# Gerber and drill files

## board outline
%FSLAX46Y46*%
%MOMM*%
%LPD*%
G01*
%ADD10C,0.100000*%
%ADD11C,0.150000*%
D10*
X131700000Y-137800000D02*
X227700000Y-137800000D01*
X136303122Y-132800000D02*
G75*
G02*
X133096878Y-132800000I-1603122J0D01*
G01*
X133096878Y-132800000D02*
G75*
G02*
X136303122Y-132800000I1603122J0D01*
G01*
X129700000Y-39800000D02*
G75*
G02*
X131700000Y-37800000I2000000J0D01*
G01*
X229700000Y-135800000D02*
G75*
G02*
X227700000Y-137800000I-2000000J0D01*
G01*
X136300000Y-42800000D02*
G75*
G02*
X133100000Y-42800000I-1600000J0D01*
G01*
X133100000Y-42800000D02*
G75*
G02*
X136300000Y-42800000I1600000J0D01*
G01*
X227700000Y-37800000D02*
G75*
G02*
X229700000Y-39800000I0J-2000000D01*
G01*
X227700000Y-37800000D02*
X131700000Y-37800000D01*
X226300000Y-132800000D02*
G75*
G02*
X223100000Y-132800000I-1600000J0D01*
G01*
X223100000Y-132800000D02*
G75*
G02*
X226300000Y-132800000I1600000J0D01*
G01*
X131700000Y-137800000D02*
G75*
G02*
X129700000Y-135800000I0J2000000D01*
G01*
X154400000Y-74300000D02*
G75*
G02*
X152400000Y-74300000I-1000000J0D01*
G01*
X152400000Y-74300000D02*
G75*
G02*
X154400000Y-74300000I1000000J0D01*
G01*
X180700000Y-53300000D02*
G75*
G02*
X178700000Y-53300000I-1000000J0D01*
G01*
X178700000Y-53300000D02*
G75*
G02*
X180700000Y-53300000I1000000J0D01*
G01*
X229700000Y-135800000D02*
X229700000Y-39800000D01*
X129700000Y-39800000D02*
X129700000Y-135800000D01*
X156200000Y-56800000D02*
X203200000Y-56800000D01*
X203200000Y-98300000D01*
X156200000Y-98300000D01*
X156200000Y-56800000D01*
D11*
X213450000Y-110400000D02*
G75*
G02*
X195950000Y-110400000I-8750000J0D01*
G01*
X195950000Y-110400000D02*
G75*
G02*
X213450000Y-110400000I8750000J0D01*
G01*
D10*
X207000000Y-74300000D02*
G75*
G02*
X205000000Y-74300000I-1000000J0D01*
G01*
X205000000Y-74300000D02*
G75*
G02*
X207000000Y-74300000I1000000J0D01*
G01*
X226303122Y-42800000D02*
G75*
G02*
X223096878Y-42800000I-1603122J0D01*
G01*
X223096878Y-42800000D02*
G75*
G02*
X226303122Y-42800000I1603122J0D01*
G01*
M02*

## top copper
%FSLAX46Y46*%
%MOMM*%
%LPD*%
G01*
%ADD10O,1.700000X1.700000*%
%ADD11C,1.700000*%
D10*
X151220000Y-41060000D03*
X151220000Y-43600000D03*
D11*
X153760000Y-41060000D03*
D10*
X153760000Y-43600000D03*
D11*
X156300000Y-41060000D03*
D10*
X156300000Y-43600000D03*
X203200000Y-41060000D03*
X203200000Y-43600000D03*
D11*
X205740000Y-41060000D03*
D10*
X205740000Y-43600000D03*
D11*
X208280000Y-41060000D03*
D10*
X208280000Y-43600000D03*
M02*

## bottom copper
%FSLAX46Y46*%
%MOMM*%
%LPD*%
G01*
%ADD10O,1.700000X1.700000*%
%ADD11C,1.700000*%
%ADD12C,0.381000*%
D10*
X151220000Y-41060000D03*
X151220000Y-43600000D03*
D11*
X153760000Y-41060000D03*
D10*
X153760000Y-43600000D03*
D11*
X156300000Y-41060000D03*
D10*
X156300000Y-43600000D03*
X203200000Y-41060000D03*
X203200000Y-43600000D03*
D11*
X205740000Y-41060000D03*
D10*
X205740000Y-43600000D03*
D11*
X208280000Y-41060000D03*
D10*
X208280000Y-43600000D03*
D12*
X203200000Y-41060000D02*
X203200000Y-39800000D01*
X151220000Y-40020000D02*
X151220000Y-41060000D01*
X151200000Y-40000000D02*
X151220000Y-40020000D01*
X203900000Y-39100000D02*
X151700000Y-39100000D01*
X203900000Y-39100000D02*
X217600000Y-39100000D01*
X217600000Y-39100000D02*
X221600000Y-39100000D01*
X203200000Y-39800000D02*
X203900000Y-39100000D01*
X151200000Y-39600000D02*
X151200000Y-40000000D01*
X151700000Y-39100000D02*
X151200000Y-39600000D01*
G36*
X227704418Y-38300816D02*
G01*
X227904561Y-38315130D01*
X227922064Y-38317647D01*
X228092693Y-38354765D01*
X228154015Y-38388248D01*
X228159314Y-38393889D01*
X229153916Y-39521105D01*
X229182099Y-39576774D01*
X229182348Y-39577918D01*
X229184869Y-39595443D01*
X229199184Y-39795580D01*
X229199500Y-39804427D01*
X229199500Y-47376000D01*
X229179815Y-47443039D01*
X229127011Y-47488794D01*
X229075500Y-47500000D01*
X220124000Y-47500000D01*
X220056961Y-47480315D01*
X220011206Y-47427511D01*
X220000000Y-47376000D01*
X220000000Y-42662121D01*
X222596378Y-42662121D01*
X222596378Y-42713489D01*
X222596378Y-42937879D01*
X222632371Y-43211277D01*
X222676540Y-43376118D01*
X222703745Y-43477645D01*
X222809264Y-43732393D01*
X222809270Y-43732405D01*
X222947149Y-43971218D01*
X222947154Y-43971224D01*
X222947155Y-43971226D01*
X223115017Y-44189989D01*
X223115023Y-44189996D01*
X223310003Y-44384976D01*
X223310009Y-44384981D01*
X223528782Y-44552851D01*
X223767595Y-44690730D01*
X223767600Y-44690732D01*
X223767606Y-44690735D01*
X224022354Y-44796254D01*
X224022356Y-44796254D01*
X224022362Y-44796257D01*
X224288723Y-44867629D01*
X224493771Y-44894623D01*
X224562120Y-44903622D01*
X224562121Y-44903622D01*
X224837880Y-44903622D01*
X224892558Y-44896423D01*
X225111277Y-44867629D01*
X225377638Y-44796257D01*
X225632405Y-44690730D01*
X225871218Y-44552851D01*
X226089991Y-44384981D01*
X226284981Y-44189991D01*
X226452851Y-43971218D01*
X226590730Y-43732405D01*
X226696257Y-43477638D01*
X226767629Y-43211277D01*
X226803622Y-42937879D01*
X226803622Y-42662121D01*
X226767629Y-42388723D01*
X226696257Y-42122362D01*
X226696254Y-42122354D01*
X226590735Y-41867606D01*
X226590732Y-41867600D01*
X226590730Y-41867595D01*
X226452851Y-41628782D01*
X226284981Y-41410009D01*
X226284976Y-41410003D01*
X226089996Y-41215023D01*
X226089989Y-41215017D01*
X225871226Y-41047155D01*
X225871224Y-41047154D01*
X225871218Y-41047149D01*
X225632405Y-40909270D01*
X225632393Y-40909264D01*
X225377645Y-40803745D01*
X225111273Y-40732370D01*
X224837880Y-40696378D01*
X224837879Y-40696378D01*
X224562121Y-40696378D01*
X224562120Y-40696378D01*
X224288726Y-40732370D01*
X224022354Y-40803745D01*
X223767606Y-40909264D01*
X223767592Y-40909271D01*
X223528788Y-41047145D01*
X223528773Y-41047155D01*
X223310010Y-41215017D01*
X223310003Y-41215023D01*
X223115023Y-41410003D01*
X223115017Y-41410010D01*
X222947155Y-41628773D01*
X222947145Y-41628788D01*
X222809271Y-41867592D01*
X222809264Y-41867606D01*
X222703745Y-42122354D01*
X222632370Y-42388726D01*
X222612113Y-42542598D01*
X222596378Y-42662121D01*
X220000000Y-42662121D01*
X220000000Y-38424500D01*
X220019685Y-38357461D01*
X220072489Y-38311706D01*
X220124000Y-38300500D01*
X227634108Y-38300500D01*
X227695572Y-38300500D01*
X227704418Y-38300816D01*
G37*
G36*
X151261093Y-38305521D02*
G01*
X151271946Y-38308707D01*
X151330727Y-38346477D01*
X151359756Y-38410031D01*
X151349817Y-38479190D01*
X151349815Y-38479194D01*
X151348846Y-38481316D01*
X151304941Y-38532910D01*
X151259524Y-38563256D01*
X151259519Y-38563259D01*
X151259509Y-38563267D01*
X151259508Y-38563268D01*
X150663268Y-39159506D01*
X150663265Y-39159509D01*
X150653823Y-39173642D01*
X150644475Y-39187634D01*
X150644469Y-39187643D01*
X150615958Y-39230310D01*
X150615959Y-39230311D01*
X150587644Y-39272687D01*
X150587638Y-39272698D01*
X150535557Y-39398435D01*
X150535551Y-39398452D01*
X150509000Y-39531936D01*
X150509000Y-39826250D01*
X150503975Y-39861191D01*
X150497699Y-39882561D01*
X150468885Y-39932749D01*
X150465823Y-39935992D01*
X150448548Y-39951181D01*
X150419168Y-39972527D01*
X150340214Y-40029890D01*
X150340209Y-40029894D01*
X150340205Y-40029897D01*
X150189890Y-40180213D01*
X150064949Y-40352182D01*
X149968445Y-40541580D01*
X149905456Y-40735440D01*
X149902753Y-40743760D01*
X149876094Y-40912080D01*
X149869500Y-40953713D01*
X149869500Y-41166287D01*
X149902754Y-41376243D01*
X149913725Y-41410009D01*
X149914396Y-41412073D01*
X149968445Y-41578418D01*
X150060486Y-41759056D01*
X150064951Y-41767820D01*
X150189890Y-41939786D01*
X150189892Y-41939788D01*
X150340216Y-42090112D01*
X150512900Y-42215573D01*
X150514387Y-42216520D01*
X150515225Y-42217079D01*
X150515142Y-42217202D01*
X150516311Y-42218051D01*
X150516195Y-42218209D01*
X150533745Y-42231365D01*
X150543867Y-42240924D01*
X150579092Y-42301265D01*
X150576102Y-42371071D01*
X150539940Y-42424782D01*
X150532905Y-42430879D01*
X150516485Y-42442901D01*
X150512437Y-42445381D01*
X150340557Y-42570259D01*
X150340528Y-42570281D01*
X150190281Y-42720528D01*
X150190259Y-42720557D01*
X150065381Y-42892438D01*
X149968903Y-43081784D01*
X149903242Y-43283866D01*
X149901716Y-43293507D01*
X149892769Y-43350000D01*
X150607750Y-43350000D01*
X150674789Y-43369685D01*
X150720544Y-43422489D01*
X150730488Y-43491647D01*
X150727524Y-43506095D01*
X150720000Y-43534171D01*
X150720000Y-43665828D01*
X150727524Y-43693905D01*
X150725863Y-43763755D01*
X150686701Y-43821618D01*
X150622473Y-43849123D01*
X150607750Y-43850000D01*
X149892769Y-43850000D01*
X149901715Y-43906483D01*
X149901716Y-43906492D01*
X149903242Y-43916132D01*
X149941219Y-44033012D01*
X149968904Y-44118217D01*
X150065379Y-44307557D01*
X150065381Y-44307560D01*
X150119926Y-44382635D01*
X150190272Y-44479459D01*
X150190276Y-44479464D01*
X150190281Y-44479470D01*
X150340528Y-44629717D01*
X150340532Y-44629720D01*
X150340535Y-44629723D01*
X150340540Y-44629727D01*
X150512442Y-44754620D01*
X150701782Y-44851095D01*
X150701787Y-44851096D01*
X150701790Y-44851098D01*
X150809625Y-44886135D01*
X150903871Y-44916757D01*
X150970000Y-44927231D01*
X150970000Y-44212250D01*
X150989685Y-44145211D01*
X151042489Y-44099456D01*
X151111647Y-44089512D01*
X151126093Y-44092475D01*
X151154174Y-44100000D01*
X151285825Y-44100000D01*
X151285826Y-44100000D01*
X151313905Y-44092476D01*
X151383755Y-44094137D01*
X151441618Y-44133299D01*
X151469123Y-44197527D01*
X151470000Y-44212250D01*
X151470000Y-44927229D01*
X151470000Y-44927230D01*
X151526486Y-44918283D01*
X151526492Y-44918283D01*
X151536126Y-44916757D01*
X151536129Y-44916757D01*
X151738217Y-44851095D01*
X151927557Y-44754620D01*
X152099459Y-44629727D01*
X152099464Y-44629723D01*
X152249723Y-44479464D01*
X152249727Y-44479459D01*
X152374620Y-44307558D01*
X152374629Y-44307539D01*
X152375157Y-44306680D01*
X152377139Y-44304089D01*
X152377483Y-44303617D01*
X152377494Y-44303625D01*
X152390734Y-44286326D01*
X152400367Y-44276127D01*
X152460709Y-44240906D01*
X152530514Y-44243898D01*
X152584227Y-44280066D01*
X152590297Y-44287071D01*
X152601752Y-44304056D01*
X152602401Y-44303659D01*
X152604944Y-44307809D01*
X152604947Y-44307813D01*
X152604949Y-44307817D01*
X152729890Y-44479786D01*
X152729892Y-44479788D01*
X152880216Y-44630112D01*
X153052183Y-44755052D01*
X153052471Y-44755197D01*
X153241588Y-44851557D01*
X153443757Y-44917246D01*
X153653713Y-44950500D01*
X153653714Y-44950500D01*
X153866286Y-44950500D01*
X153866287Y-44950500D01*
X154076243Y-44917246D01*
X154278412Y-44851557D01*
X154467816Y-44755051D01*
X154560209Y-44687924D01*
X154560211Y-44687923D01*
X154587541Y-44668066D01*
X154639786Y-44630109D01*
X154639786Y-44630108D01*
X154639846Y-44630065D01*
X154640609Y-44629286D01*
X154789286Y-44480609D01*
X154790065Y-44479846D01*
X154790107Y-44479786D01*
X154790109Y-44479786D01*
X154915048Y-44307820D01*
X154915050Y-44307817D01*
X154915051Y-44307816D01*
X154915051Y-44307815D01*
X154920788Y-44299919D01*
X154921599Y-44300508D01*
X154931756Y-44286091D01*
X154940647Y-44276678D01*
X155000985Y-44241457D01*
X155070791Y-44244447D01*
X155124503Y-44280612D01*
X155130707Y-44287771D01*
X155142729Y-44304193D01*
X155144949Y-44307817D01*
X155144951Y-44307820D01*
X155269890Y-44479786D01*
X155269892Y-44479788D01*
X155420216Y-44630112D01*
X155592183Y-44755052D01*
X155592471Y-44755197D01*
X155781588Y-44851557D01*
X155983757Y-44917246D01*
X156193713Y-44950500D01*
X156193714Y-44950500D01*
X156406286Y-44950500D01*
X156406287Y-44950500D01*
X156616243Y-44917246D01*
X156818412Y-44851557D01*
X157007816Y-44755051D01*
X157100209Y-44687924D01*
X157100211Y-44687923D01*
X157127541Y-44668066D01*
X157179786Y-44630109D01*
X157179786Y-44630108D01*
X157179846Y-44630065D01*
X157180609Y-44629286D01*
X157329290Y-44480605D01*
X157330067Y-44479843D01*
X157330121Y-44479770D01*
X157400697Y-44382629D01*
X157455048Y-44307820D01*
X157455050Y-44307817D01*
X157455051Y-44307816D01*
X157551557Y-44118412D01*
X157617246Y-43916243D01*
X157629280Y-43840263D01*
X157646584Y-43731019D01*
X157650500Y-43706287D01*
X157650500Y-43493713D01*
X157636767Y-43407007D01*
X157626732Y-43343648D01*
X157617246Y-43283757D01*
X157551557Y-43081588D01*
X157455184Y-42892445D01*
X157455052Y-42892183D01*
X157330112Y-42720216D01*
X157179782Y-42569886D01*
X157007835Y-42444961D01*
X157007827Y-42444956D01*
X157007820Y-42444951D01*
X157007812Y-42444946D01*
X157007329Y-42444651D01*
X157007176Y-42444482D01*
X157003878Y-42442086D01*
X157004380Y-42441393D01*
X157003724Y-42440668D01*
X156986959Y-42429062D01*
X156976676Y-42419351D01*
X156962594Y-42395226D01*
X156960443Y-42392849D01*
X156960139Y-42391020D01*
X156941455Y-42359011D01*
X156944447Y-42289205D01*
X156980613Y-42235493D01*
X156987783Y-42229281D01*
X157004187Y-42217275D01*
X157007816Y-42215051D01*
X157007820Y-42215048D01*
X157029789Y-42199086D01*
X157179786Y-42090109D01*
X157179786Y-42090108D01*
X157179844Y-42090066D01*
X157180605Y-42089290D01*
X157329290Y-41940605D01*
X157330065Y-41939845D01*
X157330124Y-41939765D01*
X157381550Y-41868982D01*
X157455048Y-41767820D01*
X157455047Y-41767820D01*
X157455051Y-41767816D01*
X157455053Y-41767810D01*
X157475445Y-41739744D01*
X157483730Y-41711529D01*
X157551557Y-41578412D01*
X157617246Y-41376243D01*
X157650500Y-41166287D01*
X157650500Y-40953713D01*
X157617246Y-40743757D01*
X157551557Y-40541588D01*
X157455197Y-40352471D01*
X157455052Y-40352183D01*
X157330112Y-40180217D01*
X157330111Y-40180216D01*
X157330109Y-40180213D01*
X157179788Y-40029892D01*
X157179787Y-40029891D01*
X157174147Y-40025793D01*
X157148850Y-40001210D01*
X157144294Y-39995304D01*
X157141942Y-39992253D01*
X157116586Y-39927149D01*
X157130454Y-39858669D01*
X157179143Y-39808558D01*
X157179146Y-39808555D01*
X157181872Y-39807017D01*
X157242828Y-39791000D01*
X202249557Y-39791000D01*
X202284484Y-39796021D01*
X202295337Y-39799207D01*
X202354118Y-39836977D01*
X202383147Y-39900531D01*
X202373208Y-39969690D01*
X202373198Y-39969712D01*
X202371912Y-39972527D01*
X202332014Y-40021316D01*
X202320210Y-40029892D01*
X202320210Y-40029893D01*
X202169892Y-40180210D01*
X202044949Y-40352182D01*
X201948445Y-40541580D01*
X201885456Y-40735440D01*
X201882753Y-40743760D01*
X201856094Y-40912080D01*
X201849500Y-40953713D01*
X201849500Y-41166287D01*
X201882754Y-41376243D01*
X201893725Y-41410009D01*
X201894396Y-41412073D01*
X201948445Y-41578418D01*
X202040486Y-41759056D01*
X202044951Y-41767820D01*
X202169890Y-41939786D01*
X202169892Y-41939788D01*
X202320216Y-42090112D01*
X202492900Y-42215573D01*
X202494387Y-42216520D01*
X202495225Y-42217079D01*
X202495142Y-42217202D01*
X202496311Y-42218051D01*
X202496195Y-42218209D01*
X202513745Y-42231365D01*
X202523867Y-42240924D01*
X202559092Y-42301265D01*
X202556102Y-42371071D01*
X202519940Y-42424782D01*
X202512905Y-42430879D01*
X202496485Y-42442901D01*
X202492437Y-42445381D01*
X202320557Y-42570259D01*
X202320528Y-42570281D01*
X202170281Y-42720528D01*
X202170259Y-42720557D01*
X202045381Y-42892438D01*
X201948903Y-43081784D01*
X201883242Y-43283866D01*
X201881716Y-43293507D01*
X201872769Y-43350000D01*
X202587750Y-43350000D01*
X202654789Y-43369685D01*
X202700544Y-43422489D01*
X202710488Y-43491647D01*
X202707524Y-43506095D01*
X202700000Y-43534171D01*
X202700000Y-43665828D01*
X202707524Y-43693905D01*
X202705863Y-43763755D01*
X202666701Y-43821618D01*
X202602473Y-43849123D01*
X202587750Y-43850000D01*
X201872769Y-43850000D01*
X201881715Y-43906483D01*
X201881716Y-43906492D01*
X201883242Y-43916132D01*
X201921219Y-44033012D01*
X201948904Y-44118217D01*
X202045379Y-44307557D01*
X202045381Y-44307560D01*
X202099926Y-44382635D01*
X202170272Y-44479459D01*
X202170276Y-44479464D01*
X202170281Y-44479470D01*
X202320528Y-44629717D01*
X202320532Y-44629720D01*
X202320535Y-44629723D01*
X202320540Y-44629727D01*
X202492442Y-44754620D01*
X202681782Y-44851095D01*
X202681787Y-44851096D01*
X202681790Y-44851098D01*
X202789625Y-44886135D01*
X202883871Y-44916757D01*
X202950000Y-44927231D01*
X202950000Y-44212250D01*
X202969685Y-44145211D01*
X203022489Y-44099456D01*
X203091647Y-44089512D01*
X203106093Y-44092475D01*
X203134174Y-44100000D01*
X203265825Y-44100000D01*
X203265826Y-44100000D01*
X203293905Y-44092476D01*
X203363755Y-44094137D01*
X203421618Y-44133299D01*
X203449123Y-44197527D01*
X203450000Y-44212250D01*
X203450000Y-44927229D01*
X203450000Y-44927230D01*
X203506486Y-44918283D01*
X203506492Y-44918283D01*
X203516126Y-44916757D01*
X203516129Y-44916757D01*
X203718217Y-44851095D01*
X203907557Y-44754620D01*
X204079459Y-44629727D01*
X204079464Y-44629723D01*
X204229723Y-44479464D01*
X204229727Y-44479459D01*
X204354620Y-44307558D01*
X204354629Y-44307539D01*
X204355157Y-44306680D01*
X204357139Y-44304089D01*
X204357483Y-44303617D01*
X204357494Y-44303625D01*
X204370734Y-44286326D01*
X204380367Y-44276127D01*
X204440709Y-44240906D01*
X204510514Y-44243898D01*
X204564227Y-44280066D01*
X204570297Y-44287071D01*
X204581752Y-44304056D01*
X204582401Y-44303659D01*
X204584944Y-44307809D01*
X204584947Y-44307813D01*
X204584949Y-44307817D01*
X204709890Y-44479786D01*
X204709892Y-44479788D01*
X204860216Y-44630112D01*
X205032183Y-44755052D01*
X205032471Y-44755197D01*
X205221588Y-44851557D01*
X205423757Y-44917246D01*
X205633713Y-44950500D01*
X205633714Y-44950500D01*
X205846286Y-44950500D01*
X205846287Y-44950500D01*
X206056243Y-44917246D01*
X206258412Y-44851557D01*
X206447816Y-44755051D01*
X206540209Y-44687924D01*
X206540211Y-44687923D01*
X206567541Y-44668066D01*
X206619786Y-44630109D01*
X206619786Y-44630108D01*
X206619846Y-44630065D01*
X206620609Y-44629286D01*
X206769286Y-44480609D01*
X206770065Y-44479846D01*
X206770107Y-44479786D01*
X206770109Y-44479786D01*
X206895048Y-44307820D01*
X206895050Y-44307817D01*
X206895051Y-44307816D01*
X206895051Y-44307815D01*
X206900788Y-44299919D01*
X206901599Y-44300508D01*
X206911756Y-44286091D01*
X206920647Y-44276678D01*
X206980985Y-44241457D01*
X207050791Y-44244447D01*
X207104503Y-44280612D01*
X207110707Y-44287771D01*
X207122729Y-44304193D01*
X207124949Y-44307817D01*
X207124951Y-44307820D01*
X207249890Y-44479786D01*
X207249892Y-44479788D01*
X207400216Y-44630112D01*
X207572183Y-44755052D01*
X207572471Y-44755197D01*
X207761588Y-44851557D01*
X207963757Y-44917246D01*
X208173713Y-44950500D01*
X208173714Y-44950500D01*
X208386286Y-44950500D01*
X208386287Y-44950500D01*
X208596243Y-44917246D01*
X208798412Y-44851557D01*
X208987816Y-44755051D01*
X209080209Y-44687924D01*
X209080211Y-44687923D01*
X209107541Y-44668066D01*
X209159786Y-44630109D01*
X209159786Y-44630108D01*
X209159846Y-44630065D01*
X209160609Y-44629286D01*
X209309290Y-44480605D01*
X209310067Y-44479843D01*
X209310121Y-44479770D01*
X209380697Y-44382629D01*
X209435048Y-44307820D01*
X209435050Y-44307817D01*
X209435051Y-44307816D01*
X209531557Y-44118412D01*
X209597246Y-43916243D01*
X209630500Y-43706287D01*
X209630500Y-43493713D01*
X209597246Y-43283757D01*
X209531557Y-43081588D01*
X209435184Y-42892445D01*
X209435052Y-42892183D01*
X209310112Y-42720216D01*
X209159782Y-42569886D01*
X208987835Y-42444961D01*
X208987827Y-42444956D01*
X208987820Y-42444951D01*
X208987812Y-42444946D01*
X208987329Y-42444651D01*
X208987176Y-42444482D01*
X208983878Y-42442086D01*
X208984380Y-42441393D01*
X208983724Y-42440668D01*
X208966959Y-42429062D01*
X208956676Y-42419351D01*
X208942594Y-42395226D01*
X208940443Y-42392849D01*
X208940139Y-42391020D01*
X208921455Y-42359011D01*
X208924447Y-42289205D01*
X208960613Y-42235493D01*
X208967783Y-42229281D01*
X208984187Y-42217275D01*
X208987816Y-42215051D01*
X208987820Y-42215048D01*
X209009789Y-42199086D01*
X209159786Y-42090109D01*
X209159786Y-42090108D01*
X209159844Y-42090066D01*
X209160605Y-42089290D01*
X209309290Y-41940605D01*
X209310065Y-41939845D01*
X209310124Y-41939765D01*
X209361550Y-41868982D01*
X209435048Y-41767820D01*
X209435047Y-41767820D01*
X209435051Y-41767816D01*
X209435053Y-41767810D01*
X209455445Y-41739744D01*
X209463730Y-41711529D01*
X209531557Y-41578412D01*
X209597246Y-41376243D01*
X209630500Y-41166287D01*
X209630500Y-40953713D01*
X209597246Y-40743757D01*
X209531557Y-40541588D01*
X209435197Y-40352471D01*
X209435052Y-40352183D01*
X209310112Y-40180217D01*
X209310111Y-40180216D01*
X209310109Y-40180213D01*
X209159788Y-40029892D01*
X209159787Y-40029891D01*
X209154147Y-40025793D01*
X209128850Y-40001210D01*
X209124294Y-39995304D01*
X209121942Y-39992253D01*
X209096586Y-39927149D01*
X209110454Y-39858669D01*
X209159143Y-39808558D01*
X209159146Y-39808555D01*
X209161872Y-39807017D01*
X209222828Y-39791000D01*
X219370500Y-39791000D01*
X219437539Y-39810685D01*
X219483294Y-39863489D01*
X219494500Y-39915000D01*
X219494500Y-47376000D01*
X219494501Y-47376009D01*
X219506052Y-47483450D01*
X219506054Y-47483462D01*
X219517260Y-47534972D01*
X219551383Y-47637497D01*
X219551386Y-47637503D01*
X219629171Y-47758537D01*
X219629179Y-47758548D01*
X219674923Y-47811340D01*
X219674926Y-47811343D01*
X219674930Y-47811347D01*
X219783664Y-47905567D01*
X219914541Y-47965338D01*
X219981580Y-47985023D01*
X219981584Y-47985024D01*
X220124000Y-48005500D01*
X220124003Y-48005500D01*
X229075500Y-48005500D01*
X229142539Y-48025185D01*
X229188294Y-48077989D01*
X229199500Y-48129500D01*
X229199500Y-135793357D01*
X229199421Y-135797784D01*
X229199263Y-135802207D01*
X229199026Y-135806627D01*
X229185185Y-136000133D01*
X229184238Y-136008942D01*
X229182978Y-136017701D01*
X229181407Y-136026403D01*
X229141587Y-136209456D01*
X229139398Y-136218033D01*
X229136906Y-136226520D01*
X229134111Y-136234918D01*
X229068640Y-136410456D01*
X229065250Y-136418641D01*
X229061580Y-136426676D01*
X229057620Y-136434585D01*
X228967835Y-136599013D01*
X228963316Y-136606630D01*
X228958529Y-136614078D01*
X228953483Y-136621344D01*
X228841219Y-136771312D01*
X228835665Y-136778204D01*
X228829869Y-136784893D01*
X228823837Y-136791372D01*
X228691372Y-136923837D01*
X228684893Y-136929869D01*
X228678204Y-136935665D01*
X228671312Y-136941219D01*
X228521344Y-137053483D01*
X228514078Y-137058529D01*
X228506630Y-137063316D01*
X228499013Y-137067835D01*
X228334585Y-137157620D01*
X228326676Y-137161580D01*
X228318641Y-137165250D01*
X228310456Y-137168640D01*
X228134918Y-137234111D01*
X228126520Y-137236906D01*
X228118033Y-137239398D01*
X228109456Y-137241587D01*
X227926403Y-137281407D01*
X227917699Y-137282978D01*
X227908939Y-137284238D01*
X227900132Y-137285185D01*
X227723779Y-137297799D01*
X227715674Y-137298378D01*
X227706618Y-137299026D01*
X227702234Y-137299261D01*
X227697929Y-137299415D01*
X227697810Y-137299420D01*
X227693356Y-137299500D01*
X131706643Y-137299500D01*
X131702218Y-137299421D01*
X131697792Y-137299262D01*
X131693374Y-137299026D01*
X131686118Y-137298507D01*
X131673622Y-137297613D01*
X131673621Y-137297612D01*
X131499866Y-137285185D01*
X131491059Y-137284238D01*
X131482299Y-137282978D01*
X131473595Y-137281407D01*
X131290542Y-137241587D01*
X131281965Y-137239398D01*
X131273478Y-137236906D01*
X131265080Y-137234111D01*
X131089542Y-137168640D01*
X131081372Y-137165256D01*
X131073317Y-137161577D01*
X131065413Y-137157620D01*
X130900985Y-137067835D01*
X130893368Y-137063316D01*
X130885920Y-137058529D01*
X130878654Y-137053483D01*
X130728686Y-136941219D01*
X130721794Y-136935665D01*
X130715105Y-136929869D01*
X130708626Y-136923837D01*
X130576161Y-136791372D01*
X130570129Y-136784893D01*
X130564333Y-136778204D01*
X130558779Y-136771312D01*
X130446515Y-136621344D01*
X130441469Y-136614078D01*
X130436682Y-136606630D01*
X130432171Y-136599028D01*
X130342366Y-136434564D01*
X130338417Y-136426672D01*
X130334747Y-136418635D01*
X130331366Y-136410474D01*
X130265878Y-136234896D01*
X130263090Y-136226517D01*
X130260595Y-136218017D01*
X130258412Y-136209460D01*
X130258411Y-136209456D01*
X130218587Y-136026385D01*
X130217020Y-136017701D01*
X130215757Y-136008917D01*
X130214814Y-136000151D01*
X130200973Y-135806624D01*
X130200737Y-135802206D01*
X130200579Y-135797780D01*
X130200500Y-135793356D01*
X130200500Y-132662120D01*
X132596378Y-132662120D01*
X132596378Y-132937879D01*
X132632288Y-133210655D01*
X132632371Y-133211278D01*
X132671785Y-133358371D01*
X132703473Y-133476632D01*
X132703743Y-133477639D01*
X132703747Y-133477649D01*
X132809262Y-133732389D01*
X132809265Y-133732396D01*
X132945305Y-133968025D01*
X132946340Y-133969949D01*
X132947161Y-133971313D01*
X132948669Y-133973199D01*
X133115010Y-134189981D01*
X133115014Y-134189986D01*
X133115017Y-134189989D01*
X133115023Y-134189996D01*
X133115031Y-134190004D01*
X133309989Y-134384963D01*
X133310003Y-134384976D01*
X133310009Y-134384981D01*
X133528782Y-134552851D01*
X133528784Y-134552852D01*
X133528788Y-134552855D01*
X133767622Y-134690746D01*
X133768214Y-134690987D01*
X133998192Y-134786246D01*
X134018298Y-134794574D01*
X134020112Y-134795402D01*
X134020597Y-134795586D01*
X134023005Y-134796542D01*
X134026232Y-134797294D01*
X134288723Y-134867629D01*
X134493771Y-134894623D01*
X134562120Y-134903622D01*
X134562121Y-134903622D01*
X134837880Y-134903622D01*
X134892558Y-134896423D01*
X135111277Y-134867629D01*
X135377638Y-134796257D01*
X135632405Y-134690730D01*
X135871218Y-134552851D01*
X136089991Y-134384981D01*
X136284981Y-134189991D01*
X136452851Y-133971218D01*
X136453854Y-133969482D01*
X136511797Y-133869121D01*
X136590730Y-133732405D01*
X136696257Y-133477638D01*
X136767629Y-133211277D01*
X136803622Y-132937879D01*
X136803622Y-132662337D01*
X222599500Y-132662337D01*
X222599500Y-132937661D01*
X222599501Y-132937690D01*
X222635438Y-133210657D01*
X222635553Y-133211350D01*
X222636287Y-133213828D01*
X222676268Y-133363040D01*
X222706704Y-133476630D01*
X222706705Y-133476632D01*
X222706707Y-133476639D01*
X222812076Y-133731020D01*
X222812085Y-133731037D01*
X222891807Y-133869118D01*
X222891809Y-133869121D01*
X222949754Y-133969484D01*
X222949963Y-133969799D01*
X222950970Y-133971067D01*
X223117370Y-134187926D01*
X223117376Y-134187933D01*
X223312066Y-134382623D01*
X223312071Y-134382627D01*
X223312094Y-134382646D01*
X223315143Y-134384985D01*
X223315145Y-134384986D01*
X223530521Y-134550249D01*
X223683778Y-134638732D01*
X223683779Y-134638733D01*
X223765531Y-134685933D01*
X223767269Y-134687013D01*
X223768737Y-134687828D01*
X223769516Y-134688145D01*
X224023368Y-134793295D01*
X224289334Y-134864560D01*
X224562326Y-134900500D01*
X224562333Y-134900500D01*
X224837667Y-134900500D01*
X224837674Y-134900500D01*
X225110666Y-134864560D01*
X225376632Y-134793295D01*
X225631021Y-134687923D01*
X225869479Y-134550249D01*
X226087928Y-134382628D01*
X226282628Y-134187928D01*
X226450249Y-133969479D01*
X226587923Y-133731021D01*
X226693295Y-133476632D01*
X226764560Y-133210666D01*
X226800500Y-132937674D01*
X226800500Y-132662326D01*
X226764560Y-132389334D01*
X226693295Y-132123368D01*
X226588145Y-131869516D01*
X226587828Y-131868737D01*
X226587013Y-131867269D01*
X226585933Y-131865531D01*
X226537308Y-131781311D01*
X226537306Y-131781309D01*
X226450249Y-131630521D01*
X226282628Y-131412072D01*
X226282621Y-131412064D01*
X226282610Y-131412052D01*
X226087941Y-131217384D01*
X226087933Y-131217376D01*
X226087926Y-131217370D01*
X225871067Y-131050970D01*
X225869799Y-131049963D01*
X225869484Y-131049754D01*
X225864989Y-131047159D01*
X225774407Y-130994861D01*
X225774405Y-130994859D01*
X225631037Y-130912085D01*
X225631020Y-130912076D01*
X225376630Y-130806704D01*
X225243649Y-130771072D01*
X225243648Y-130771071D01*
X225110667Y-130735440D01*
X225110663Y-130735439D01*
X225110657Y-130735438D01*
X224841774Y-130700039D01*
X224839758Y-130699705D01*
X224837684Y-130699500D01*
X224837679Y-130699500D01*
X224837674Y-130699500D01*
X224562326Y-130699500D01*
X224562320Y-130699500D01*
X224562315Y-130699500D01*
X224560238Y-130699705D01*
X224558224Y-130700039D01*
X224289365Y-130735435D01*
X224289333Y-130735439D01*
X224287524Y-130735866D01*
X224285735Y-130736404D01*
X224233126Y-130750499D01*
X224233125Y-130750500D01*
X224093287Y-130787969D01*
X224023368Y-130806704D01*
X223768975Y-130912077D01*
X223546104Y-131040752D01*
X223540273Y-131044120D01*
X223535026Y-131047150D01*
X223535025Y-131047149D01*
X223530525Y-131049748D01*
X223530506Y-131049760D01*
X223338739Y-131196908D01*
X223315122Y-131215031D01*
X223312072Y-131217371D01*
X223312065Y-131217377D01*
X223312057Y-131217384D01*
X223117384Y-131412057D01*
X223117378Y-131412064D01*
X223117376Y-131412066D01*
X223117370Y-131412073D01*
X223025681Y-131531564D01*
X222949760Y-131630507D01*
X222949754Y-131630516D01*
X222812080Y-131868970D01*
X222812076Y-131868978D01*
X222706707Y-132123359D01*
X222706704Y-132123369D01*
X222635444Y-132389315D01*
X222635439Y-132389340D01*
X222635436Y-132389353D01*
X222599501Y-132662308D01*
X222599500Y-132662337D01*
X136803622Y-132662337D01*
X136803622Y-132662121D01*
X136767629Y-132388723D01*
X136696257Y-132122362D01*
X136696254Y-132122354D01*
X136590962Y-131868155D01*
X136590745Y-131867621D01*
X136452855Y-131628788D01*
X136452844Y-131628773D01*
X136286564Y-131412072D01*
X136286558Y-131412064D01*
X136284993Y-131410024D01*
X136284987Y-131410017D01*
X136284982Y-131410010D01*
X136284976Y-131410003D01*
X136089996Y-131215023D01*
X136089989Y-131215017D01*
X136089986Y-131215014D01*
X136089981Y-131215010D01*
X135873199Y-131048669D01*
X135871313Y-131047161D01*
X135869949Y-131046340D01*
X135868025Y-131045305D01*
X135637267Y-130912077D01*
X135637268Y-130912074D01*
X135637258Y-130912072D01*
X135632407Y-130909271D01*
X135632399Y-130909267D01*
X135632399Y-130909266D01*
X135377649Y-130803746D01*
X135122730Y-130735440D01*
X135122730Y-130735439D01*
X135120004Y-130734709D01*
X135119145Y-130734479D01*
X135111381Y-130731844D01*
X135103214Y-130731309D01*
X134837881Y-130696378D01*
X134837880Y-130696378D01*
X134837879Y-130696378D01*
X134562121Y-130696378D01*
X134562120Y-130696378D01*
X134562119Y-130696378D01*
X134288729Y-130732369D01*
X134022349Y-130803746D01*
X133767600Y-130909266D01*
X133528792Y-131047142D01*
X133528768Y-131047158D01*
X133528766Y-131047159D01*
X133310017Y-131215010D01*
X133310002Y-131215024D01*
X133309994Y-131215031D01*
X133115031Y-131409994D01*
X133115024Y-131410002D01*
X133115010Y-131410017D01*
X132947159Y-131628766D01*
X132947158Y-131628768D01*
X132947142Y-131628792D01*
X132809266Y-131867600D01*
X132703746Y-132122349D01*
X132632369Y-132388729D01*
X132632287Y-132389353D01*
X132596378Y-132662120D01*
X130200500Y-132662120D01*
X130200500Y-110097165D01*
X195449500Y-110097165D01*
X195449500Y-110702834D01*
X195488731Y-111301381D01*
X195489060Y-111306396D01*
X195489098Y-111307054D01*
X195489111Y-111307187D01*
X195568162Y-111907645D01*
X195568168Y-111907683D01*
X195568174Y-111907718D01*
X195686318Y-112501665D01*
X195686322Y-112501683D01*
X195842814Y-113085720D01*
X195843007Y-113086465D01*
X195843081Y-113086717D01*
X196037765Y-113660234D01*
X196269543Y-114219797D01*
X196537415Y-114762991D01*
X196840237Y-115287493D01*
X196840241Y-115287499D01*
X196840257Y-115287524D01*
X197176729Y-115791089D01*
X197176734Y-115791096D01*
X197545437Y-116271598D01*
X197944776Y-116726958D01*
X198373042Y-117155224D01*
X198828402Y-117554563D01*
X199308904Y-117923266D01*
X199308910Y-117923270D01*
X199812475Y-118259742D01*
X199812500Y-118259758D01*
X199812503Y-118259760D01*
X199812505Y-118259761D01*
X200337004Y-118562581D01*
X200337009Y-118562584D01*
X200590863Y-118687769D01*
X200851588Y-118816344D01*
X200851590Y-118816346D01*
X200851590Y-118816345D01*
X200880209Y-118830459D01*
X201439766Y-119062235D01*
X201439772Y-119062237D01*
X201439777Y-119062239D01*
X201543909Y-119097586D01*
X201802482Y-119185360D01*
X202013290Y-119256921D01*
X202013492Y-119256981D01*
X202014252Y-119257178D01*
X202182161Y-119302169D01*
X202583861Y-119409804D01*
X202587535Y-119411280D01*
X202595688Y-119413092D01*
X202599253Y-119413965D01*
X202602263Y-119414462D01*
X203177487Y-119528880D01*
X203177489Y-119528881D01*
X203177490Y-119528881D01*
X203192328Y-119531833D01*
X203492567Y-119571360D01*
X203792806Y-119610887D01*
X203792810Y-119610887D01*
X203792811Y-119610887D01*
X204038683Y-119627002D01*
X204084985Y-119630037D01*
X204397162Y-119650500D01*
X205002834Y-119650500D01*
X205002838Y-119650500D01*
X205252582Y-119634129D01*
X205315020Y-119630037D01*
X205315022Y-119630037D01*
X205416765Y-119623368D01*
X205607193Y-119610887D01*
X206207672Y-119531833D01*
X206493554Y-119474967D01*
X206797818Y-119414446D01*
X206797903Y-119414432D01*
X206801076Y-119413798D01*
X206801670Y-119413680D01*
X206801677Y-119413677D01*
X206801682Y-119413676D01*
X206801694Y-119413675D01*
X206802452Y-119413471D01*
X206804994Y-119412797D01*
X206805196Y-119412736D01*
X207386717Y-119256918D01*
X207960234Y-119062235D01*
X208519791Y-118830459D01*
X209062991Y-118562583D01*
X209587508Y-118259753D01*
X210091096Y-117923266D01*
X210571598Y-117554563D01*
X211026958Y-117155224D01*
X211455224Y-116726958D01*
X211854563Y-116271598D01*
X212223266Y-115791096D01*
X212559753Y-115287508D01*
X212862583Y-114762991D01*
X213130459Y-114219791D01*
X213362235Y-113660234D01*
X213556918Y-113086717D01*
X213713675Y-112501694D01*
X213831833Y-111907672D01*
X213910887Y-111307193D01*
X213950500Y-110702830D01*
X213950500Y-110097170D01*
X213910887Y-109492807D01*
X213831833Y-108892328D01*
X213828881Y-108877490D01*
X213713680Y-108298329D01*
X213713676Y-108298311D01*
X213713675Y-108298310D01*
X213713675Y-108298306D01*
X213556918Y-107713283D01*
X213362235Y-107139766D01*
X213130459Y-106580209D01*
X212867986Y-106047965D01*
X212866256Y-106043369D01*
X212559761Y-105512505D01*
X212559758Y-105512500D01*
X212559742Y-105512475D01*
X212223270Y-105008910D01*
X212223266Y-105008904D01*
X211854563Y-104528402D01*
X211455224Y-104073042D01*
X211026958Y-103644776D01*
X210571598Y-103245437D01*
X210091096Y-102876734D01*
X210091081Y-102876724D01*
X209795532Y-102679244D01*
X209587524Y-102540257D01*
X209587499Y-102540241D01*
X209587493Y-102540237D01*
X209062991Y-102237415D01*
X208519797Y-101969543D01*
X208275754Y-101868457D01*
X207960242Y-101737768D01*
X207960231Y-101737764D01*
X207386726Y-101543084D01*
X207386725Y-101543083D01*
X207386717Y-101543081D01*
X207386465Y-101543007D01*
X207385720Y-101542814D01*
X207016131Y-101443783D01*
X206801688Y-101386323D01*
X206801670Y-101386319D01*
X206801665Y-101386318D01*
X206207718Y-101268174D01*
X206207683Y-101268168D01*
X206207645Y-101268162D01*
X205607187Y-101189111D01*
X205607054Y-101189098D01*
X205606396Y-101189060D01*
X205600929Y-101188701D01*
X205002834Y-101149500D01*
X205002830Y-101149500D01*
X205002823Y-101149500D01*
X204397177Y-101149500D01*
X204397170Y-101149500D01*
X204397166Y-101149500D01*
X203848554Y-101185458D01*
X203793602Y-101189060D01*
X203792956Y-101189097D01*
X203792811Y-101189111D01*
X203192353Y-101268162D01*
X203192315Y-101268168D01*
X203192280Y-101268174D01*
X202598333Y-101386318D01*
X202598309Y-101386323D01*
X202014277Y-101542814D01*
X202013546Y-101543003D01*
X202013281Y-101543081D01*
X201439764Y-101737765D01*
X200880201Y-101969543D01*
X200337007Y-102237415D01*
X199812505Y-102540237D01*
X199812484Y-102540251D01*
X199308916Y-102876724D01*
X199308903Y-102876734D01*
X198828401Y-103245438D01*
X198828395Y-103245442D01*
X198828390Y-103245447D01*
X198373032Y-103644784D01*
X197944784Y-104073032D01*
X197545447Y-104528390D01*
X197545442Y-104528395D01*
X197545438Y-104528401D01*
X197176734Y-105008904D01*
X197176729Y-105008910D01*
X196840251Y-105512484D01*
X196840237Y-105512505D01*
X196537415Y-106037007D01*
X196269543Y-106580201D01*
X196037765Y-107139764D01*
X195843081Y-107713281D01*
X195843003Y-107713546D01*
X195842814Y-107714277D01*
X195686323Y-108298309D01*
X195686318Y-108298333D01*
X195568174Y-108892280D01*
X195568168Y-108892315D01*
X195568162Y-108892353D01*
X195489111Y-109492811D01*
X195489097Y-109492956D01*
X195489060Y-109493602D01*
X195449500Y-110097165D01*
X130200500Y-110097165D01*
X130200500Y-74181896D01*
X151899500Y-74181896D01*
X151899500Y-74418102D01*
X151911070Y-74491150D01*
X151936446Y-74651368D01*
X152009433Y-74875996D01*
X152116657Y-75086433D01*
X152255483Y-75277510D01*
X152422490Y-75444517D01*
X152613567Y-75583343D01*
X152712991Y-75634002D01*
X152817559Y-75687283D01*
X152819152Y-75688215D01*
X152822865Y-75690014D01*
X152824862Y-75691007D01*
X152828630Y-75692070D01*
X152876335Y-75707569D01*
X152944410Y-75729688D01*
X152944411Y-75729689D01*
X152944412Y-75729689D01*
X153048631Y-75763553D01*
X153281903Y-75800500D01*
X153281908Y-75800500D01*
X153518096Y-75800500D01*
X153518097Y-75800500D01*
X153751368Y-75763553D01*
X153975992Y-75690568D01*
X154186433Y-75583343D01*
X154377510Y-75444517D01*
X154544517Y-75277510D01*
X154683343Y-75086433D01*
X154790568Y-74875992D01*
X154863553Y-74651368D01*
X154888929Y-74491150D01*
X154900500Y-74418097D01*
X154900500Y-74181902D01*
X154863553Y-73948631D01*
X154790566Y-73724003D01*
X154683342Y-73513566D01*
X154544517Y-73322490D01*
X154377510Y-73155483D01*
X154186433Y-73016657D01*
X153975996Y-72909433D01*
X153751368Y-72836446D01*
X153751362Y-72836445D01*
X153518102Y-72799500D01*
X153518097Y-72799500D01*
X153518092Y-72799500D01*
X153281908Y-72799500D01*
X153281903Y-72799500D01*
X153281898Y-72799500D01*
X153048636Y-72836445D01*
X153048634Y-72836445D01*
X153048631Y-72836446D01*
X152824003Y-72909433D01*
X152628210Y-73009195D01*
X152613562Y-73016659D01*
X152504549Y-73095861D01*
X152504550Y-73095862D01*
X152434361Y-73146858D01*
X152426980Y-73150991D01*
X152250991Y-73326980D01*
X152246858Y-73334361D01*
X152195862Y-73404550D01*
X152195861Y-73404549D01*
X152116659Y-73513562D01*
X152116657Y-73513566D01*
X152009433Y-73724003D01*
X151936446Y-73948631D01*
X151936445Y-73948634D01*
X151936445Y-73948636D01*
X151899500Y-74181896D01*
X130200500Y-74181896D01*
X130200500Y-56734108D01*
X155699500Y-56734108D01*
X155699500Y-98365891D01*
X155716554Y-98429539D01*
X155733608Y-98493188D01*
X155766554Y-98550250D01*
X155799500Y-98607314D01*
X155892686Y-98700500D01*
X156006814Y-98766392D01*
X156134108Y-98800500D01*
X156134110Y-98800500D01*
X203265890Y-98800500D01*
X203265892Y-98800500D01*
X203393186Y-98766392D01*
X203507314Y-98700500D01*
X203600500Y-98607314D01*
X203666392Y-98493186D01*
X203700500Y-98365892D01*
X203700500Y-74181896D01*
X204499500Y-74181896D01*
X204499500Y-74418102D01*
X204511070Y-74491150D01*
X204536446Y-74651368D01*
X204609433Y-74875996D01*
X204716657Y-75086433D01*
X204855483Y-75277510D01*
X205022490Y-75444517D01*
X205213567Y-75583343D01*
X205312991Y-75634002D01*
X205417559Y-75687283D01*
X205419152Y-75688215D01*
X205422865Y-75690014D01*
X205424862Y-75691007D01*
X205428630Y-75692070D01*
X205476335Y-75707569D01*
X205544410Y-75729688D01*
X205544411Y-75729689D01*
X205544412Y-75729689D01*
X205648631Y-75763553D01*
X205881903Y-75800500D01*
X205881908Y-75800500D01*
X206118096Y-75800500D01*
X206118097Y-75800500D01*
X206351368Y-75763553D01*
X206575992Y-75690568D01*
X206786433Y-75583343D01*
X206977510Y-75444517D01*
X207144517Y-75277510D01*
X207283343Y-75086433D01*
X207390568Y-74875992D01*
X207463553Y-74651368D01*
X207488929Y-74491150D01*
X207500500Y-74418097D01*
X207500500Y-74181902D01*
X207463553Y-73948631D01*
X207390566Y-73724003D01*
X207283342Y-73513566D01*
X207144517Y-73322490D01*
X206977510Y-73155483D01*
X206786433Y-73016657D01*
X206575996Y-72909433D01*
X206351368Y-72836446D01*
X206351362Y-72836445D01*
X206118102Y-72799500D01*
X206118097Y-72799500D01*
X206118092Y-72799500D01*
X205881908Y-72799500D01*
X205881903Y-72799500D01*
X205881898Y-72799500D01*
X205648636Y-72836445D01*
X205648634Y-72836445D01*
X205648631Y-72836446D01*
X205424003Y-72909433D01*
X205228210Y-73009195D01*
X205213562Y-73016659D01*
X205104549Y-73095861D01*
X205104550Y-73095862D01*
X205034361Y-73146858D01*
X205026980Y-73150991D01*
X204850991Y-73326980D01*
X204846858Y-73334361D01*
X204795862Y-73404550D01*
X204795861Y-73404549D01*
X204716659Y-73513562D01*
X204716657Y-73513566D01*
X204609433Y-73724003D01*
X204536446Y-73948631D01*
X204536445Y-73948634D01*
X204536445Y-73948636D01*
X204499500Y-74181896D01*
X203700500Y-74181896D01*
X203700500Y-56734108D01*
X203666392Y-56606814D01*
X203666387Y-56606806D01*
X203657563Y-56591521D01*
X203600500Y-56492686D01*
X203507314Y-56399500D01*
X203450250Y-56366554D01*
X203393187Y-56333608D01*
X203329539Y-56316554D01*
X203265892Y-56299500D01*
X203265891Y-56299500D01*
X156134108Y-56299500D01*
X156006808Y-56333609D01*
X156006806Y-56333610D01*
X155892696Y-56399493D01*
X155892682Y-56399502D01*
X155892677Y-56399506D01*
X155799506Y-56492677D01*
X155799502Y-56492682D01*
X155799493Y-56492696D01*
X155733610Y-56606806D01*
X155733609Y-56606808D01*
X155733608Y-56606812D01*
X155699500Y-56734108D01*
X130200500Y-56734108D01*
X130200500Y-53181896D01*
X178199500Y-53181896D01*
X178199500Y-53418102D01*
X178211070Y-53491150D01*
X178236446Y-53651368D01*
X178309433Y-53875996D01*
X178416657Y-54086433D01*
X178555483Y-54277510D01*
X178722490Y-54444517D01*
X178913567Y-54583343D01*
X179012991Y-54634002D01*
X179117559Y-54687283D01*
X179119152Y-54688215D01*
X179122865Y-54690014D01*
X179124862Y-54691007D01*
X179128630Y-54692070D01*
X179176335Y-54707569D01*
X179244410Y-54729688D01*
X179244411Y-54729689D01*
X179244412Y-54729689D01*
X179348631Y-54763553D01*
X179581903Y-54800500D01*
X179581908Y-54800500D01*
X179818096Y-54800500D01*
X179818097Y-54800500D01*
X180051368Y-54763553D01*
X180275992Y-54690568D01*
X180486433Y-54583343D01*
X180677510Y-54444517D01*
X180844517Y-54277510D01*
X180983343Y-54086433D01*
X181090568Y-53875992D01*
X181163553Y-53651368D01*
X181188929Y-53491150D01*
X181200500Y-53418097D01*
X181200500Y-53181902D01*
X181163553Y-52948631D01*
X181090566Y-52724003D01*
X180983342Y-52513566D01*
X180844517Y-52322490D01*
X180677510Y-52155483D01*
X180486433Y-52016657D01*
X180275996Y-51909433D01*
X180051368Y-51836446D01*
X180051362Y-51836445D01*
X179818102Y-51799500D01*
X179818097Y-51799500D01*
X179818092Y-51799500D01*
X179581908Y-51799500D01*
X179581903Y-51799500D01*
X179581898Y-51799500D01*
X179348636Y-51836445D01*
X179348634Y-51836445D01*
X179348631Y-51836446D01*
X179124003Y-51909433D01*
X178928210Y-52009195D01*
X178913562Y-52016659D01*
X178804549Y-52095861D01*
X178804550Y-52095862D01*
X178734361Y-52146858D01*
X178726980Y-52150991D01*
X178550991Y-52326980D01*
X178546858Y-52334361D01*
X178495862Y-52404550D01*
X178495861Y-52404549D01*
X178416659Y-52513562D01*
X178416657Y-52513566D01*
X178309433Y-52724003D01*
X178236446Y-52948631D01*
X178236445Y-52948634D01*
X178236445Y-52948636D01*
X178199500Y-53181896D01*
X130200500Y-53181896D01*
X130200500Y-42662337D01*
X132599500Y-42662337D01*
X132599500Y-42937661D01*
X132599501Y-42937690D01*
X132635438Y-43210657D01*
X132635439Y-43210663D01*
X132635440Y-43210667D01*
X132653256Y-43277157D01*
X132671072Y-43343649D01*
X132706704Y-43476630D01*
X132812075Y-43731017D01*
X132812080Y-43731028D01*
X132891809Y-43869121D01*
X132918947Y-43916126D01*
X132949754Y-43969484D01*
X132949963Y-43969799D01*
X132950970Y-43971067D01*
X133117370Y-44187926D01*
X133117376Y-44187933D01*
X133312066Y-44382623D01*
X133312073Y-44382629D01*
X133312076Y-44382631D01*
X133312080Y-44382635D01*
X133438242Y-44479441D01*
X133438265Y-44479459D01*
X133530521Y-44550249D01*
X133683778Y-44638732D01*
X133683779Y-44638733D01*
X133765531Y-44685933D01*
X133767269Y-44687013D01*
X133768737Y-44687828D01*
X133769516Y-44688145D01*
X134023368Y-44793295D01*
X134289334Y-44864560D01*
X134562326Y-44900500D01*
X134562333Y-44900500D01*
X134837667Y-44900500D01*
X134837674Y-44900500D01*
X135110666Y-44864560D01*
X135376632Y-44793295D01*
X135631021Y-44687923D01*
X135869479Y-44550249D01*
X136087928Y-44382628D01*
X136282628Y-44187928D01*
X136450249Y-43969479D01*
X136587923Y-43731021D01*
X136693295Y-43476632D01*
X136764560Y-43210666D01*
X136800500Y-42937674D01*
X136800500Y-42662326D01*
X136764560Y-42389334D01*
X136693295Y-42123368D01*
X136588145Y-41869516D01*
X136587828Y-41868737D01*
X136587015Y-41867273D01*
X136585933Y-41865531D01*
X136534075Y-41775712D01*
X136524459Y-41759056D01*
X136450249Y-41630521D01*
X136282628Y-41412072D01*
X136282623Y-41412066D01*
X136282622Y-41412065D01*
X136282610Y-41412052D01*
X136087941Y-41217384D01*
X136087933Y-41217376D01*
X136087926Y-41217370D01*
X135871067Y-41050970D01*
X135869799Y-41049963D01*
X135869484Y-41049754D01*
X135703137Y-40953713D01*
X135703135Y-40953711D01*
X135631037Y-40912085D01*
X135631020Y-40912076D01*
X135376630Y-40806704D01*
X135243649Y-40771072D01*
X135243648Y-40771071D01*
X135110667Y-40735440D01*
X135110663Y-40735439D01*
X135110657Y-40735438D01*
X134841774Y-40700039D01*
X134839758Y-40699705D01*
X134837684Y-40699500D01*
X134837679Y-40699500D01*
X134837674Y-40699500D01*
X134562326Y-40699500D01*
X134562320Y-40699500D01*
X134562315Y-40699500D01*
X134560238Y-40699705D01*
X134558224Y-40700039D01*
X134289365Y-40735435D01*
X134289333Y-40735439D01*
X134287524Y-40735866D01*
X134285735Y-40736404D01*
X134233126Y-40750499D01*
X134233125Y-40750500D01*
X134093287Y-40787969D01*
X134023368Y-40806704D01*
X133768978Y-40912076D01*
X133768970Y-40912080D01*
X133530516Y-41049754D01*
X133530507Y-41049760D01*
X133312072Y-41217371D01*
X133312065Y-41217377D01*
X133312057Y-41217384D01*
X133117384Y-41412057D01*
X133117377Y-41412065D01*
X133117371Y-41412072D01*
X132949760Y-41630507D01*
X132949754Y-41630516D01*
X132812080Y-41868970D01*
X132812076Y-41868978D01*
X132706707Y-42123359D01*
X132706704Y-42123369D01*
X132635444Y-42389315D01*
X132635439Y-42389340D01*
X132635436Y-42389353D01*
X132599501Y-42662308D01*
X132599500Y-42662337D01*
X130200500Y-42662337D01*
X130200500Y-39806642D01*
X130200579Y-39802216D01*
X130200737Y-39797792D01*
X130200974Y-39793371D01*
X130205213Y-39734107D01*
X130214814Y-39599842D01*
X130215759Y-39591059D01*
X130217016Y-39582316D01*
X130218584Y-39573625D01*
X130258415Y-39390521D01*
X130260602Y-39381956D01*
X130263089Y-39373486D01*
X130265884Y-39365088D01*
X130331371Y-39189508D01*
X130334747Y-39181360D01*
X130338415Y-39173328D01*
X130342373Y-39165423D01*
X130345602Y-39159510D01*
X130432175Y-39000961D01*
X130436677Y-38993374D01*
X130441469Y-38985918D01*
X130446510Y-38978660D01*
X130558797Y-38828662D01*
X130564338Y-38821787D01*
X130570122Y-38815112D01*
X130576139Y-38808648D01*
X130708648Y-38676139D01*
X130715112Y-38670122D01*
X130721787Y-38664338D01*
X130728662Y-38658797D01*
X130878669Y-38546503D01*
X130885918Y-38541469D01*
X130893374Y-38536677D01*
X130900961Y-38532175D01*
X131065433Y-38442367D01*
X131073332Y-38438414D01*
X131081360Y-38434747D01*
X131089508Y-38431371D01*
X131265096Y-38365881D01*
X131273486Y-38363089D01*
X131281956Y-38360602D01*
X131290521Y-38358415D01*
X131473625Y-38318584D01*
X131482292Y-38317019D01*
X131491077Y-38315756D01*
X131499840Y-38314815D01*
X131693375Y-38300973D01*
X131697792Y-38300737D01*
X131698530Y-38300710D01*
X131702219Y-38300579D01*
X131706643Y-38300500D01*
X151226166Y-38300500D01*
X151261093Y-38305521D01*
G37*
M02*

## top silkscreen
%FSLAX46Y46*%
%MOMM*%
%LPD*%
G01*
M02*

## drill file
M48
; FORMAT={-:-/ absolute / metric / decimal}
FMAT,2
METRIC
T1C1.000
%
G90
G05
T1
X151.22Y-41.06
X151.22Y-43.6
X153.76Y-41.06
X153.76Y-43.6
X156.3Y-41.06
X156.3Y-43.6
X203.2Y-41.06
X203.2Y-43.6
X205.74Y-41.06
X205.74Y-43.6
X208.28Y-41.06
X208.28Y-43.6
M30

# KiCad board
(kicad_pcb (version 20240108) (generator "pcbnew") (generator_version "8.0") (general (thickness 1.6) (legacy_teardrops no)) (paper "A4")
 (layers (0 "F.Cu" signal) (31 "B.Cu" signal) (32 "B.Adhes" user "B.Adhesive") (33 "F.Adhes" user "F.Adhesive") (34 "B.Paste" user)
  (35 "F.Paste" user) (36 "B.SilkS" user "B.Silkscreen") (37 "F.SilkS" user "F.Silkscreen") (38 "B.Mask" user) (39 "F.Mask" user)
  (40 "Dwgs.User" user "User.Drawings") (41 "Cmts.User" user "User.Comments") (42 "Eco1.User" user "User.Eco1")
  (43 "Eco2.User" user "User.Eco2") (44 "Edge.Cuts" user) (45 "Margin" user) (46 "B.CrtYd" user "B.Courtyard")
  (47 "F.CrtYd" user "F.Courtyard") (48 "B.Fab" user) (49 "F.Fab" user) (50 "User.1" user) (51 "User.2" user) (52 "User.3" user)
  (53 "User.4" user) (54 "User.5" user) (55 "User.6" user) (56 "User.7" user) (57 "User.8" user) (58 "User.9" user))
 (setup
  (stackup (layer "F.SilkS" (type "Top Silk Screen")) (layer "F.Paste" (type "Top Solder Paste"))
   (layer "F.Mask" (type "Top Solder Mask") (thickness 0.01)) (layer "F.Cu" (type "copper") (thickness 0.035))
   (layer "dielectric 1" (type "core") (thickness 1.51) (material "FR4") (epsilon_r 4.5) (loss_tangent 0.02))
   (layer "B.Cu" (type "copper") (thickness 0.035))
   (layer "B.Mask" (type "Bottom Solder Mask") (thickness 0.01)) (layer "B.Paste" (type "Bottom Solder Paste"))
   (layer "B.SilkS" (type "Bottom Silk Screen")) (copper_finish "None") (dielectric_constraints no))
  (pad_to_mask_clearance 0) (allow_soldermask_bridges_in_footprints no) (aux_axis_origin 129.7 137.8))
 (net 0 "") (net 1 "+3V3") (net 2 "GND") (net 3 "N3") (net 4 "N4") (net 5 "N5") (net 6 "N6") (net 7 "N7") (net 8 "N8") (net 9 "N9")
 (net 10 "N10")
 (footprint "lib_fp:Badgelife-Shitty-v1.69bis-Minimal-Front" (layer "F.Cu") (at 153.76 42.33)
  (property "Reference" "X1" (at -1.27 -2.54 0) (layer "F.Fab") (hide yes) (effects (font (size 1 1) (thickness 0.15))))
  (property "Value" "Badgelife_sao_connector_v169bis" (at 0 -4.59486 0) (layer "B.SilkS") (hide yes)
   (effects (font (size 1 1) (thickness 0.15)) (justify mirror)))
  (pad "1" thru_hole oval (at -2.54 -1.27) (size 1.7 1.7) (drill 1) (layers "*.Cu" "B.Mask") (remove_unused_layers no) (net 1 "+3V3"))
  (pad "2" thru_hole oval (at -2.54 1.27) (size 1.7 1.7) (drill 1) (layers "*.Cu" "B.Mask") (remove_unused_layers no) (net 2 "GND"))
  (pad "3" thru_hole circle (at 0 -1.27) (size 1.7 1.7) (drill 1) (layers "*.Cu" "B.Mask") (remove_unused_layers no) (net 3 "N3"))
  (pad "4" thru_hole oval (at 0 1.27) (size 1.7 1.7) (drill 1) (layers "*.Cu" "B.Mask") (remove_unused_layers no) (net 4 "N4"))
  (pad "5" thru_hole circle (at 2.54 -1.27) (size 1.7 1.7) (drill 1) (layers "*.Cu" "B.Mask") (remove_unused_layers no) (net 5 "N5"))
  (pad "6" thru_hole oval (at 2.54 1.27) (size 1.7 1.7) (drill 1) (layers "*.Cu" "B.Mask") (remove_unused_layers no) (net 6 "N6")))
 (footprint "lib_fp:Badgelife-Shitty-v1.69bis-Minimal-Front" (layer "F.Cu") (at 205.74 42.33)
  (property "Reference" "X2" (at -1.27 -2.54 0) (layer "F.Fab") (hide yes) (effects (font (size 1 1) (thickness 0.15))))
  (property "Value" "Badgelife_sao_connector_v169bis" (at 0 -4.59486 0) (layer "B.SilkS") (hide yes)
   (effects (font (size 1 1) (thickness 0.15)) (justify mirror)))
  (pad "1" thru_hole oval (at -2.54 -1.27) (size 1.7 1.7) (drill 1) (layers "*.Cu" "B.Mask") (remove_unused_layers no) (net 1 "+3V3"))
  (pad "2" thru_hole oval (at -2.54 1.27) (size 1.7 1.7) (drill 1) (layers "*.Cu" "B.Mask") (remove_unused_layers no) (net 2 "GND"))
  (pad "3" thru_hole circle (at 0 -1.27) (size 1.7 1.7) (drill 1) (layers "*.Cu" "B.Mask") (remove_unused_layers no) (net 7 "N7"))
  (pad "4" thru_hole oval (at 0 1.27) (size 1.7 1.7) (drill 1) (layers "*.Cu" "B.Mask") (remove_unused_layers no) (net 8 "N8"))
  (pad "5" thru_hole circle (at 2.54 -1.27) (size 1.7 1.7) (drill 1) (layers "*.Cu" "B.Mask") (remove_unused_layers no) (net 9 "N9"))
  (pad "6" thru_hole oval (at 2.54 1.27) (size 1.7 1.7) (drill 1) (layers "*.Cu" "B.Mask") (remove_unused_layers no) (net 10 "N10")))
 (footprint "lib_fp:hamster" (layer "B.Cu") (at 135.1 118.3 180)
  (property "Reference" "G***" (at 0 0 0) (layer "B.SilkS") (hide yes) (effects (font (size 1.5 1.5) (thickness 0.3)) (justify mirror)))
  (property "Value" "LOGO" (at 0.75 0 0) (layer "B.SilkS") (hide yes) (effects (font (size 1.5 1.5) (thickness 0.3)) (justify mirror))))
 (gr_line (start 131.7 137.8) (end 227.7 137.8) (stroke (width 0.1) (type default)) (layer "Edge.Cuts"))
 (gr_circle (center 134.7 132.8) (end 136.3 132.9) (stroke (width 0.1) (type default)) (fill none) (layer "Edge.Cuts"))
 (gr_arc (start 129.7 39.8) (mid 130.285786 38.385786) (end 131.7 37.8) (stroke (width 0.1) (type default)) (layer "Edge.Cuts"))
 (gr_arc (start 229.7 135.8) (mid 229.114214 137.214214) (end 227.7 137.8) (stroke (width 0.1) (type default)) (layer "Edge.Cuts"))
 (gr_circle (center 134.7 42.8) (end 136.3 42.8) (stroke (width 0.1) (type default)) (fill none) (layer "Edge.Cuts"))
 (gr_arc (start 227.7 37.8) (mid 229.114214 38.385786) (end 229.7 39.8) (stroke (width 0.1) (type default)) (layer "Edge.Cuts"))
 (gr_line (start 227.7 37.8) (end 131.7 37.8) (stroke (width 0.1) (type default)) (layer "Edge.Cuts"))
 (gr_circle (center 224.7 132.8) (end 226.3 132.8) (stroke (width 0.1) (type default)) (fill none) (layer "Edge.Cuts"))
 (gr_arc (start 131.7 137.8) (mid 130.285786 137.214214) (end 129.7 135.8) (stroke (width 0.1) (type default)) (layer "Edge.Cuts"))
 (gr_circle (center 153.4 74.3) (end 154.4 74.3) (stroke (width 0.1) (type default)) (fill none) (layer "Edge.Cuts"))
 (gr_circle (center 179.7 53.3) (end 180.7 53.3) (stroke (width 0.1) (type default)) (fill none) (layer "Edge.Cuts"))
 (gr_line (start 229.7 135.8) (end 229.7 39.8) (stroke (width 0.1) (type default)) (layer "Edge.Cuts"))
 (gr_line (start 129.7 39.8) (end 129.7 135.8) (stroke (width 0.1) (type default)) (layer "Edge.Cuts"))
 (gr_rect (start 156.2 56.8) (end 203.2 98.3) (stroke (width 0.1) (type default)) (fill none) (layer "Edge.Cuts"))
 (gr_circle (center 204.7 110.4) (end 213.45 110.4) (stroke (width 0.15) (type default)) (fill none) (layer "Edge.Cuts"))
 (gr_circle (center 206 74.3) (end 207 74.3) (stroke (width 0.1) (type default)) (fill none) (layer "Edge.Cuts"))
 (gr_circle (center 224.7 42.8) (end 226.3 42.9) (stroke (width 0.1) (type default)) (fill none) (layer "Edge.Cuts"))
 (segment (start 203.2 41.06) (end 203.2 39.8) (width 0.381) (layer "B.Cu") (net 1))
 (segment (start 151.22 40.02) (end 151.22 41.06) (width 0.381) (layer "B.Cu") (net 1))
 (segment (start 151.2 40) (end 151.22 40.02) (width 0.381) (layer "B.Cu") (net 1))
 (segment (start 203.9 39.1) (end 151.7 39.1) (width 0.381) (layer "B.Cu") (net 1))
 (segment (start 203.9 39.1) (end 217.6 39.1) (width 0.381) (layer "B.Cu") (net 1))
 (segment (start 217.6 39.1) (end 221.6 39.1) (width 0.381) (layer "B.Cu") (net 1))
 (segment (start 203.2 39.8) (end 203.9 39.1) (width 0.381) (layer "B.Cu") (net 1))
 (segment (start 151.2 39.6) (end 151.2 40) (width 0.381) (layer "B.Cu") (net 1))
 (segment (start 151.7 39.1) (end 151.2 39.6) (width 0.381) (layer "B.Cu") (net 1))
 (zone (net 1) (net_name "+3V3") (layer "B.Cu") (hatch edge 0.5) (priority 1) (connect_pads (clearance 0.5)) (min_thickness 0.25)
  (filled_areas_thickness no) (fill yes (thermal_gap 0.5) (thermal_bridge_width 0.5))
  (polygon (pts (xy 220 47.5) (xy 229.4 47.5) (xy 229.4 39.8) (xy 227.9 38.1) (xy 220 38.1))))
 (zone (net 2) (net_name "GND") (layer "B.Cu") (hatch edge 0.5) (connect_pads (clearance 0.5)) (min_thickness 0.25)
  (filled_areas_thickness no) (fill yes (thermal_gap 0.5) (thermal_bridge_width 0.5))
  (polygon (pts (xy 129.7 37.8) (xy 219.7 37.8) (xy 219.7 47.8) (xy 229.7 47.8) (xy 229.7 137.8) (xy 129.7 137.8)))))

